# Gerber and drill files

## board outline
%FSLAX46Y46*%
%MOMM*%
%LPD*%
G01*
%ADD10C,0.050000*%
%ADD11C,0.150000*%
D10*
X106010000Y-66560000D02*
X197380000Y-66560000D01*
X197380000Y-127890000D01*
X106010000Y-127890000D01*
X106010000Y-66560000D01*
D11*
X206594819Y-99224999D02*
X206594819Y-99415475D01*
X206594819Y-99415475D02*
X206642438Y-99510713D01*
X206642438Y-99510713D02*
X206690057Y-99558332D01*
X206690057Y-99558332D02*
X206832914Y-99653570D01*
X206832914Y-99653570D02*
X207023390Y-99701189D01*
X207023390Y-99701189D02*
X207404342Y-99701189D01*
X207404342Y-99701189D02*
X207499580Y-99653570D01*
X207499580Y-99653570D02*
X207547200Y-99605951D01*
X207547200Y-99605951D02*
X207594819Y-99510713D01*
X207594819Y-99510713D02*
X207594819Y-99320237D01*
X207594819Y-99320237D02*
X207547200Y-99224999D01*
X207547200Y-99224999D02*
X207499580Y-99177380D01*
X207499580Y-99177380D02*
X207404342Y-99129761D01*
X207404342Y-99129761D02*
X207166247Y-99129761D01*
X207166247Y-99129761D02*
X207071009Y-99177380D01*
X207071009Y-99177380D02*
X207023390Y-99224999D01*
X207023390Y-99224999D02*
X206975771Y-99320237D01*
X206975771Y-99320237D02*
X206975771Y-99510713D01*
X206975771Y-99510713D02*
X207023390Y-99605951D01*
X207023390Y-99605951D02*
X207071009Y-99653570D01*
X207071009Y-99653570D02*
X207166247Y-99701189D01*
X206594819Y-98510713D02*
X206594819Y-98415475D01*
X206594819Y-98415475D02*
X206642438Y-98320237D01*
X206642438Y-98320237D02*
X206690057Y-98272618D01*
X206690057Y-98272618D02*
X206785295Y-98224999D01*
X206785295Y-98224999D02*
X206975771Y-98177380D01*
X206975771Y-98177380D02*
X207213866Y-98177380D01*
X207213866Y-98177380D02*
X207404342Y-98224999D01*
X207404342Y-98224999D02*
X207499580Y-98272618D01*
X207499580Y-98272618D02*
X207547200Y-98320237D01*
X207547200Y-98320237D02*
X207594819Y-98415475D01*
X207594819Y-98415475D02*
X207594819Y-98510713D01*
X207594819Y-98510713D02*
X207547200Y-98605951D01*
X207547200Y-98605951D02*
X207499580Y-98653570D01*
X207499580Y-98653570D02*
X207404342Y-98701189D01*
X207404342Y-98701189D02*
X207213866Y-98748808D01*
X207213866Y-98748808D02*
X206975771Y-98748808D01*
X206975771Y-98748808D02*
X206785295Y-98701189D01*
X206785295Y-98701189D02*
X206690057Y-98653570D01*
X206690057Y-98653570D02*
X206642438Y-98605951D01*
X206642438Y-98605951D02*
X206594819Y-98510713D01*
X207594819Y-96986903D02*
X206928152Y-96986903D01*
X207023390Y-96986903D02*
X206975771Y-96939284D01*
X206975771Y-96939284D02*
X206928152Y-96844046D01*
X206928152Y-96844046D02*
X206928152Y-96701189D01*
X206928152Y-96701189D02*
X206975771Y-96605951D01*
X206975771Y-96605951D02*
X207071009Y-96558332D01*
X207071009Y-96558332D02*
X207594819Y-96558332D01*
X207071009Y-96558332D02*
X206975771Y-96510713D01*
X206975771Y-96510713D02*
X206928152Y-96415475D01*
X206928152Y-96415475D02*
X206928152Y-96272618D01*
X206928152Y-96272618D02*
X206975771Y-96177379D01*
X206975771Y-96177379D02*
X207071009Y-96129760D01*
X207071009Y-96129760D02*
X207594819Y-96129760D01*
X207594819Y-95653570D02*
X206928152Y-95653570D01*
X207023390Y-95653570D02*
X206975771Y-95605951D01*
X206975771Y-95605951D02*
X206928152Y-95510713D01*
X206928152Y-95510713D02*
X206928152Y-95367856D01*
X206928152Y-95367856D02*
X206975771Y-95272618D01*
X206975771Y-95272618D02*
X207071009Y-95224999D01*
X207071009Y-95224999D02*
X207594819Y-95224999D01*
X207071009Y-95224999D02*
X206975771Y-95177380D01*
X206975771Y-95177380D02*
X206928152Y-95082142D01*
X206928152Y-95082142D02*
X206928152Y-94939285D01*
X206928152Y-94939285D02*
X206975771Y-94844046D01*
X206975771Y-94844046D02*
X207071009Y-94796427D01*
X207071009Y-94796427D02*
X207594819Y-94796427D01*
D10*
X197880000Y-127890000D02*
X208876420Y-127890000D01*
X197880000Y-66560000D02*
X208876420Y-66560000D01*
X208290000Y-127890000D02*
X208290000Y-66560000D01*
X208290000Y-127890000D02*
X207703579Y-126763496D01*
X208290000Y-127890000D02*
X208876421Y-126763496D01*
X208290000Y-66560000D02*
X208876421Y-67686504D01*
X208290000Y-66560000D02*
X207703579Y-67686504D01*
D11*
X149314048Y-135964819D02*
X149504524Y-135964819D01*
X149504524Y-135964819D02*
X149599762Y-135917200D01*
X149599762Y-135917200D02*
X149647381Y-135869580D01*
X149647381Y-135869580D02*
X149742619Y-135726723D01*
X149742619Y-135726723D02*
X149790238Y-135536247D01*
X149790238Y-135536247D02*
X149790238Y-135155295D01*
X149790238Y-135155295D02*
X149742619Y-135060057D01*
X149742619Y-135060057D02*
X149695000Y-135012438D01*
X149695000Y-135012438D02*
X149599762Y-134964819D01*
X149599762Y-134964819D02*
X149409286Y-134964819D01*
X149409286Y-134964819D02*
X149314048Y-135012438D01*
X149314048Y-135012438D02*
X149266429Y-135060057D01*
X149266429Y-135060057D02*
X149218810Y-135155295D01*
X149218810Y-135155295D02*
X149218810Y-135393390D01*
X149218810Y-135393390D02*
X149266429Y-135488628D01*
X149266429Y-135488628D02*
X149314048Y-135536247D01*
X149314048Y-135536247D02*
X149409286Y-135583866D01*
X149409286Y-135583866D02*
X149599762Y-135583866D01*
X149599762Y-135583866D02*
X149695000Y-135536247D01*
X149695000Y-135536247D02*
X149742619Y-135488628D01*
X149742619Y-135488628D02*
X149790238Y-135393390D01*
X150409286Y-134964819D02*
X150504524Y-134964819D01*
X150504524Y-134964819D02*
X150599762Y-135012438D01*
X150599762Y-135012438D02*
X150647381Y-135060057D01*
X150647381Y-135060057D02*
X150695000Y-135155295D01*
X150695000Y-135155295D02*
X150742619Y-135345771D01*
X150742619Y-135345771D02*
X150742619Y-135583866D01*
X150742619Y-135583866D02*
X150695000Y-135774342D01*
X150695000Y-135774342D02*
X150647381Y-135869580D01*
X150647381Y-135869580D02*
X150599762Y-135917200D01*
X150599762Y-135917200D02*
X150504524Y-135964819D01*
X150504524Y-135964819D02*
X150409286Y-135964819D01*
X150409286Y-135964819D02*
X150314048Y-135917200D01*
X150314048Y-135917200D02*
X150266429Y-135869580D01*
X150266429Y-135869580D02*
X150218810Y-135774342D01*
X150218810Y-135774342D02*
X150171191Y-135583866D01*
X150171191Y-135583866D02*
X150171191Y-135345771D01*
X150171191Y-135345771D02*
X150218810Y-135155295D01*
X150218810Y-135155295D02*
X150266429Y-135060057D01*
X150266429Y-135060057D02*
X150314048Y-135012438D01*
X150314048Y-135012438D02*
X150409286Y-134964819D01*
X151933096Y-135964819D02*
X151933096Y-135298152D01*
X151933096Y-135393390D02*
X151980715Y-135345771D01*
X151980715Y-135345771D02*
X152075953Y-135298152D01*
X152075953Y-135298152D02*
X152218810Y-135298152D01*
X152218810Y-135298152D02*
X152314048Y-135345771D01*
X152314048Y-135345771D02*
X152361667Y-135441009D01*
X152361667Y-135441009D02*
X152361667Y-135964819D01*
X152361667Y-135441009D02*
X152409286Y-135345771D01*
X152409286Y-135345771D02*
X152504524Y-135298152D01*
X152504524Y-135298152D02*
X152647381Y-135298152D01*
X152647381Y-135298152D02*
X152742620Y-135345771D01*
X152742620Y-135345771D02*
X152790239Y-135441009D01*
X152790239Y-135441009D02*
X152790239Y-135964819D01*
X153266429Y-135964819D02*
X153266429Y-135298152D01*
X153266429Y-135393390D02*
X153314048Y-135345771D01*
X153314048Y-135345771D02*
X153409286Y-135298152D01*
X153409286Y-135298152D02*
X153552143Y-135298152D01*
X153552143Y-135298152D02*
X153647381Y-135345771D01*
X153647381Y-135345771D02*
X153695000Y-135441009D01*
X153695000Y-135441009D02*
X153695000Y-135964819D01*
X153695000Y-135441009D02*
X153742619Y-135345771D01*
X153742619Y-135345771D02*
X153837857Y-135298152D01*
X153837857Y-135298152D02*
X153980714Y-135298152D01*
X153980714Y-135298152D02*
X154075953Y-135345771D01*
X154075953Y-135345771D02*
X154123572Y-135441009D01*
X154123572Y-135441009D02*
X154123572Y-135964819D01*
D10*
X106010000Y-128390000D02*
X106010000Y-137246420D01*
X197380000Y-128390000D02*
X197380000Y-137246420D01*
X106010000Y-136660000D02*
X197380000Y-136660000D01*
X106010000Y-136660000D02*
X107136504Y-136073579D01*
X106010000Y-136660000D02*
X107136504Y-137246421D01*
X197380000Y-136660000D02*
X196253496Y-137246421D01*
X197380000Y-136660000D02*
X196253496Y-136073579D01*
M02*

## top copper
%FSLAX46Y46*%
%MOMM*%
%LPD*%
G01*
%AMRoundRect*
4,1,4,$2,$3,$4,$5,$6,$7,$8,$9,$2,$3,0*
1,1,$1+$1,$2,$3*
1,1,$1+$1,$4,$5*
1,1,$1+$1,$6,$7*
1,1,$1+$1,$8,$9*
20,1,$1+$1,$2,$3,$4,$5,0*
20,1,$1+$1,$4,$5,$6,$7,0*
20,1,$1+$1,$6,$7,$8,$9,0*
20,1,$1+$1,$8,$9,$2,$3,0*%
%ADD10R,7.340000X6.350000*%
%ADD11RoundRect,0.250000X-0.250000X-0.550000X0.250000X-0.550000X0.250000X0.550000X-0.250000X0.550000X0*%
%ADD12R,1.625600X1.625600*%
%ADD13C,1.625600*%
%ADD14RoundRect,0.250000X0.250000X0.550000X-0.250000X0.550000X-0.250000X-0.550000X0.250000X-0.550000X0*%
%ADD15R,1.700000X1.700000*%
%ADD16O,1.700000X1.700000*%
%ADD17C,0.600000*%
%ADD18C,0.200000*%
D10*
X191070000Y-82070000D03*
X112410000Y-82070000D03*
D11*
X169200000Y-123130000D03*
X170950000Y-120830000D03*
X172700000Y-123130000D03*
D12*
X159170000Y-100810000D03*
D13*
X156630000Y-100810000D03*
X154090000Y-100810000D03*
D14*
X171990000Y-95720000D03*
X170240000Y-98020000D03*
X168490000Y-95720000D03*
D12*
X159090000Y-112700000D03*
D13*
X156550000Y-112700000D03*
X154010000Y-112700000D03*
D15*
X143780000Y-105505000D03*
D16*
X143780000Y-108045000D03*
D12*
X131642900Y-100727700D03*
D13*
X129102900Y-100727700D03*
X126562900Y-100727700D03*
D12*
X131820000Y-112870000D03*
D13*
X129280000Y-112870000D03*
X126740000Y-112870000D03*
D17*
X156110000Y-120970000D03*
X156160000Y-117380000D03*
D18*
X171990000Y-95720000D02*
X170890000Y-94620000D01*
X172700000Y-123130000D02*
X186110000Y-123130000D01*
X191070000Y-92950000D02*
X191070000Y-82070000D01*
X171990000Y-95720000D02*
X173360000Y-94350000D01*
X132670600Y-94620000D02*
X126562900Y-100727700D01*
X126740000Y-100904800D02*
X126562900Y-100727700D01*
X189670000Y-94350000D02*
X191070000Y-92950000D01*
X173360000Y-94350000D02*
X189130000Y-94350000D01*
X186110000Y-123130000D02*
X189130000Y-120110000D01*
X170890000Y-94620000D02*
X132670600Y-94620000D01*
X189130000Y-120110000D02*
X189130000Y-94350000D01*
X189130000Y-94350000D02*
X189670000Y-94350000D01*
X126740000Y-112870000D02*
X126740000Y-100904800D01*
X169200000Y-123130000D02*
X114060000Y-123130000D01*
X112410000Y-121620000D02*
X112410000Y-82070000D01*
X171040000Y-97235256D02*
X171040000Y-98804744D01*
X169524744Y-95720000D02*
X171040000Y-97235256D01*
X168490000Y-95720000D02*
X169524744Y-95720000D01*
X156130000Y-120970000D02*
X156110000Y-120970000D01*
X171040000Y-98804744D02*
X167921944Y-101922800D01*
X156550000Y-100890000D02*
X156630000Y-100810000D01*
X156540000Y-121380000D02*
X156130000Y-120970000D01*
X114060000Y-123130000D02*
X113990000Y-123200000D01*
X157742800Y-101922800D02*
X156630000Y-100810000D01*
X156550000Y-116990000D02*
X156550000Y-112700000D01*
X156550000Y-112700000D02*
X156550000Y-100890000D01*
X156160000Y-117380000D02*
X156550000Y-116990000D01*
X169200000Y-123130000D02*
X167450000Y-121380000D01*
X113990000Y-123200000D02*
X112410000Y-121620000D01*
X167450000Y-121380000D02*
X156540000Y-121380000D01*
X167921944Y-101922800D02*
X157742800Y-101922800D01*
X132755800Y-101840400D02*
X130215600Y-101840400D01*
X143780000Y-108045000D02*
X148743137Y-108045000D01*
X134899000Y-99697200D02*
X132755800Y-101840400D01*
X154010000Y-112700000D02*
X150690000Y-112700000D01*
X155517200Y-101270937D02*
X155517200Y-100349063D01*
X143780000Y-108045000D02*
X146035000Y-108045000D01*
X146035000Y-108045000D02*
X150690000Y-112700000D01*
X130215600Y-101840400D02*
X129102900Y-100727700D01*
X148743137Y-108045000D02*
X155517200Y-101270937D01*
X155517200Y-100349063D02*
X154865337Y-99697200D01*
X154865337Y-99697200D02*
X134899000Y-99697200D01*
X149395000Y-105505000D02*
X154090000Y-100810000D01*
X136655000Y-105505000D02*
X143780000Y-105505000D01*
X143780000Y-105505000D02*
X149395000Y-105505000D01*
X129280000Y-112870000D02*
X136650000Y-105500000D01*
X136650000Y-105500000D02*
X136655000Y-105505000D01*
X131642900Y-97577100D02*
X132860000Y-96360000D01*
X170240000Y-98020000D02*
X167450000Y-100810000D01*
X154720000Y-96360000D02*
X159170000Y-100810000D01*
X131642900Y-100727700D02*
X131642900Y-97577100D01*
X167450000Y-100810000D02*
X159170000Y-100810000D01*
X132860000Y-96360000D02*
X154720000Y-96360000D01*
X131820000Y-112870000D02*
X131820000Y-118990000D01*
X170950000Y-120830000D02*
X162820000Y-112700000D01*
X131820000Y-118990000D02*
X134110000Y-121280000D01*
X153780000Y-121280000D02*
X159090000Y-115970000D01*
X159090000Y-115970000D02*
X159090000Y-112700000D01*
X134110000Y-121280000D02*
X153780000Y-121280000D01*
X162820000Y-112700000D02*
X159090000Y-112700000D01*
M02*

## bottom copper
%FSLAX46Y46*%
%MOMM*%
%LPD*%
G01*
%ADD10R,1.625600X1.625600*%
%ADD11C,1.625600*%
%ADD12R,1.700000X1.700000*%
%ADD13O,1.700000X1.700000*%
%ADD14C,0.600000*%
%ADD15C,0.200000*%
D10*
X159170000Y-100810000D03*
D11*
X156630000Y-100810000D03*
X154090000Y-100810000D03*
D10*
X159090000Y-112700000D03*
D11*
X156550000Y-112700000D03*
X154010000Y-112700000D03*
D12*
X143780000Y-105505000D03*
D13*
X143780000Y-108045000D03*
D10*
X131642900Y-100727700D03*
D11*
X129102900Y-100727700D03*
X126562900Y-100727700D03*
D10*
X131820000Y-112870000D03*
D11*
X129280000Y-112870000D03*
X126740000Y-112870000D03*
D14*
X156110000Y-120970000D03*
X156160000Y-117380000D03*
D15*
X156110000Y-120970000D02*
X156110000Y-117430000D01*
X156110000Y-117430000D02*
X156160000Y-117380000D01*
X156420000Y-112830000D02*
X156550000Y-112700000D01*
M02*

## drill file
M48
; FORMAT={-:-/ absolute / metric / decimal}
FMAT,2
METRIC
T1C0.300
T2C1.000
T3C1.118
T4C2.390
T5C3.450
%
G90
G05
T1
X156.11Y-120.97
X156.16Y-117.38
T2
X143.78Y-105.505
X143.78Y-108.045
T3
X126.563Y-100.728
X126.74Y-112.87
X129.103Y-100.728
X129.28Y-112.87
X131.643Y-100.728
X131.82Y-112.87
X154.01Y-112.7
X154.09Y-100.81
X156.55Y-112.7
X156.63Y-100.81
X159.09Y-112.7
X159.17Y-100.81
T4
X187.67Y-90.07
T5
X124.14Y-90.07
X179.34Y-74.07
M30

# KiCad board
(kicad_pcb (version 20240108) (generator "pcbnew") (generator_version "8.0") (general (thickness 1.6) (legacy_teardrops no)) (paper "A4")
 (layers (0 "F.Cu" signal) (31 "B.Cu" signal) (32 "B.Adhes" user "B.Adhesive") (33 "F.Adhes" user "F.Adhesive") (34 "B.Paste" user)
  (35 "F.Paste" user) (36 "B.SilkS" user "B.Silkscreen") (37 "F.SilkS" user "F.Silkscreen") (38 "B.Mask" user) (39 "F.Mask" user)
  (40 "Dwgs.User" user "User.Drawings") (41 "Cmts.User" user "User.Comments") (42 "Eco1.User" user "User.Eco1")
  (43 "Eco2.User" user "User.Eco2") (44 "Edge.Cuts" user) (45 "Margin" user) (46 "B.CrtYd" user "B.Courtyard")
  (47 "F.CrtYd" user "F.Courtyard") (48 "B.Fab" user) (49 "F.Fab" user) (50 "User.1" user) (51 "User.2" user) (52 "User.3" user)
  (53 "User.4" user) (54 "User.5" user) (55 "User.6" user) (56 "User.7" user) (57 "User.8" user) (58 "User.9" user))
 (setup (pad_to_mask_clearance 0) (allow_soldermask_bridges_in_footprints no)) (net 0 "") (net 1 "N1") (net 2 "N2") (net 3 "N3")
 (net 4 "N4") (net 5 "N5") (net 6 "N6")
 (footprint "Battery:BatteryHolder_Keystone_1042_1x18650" (layer "F.Cu") (at 151.74 82.07 180)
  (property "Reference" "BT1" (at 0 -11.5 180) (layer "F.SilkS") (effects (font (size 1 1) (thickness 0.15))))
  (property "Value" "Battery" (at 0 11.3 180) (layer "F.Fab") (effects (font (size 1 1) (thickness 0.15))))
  (pad "" np_thru_hole circle (at -35.93 -8 180) (size 2.39 2.39) (drill 2.39) (layers "*.Cu" "*.Mask"))
  (pad "" np_thru_hole circle (at -27.6 8 180) (size 3.45 3.45) (drill 3.45) (layers "*.Cu" "*.Mask"))
  (pad "" np_thru_hole circle (at 27.6 -8 180) (size 3.45 3.45) (drill 3.45) (layers "*.Cu" "*.Mask"))
  (pad "1" smd rect (at -39.33 0 180) (size 7.34 6.35) (layers "F.Cu" "F.Paste" "F.Mask") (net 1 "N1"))
  (pad "2" smd rect (at 39.33 0 180) (size 7.34 6.35) (layers "F.Cu" "F.Paste" "F.Mask") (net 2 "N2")))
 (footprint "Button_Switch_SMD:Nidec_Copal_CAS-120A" (layer "F.Cu") (at 170.95 121.98 90)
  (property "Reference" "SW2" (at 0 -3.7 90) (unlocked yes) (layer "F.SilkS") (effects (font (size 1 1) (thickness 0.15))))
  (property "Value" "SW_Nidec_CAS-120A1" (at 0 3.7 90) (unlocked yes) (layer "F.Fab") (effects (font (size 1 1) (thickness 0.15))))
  (pad "1" smd roundrect (at -1.15 -1.75) (size 1 1.6) (layers "F.Cu" "F.Paste" "F.Mask") (roundrect_rratio 0.25) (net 2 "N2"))
  (pad "2" smd roundrect (at 1.15 0) (size 1 1.6) (layers "F.Cu" "F.Paste" "F.Mask") (roundrect_rratio 0.25) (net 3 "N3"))
  (pad "3" smd roundrect (at -1.15 1.75) (size 1 1.6) (layers "F.Cu" "F.Paste" "F.Mask") (roundrect_rratio 0.25) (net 1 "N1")))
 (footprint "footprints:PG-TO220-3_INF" (layer "F.Cu") (at 159.17 100.81 180)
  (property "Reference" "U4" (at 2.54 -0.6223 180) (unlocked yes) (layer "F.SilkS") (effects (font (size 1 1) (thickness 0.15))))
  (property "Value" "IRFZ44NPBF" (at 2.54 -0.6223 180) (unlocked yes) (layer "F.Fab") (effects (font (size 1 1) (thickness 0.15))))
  (pad "1" thru_hole rect (at 0 0 180) (size 1.6256 1.6256) (drill 1.1176) (layers "*.Cu" "*.Mask") (remove_unused_layers no) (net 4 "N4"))
  (pad "2" thru_hole circle (at 2.54 0 180) (size 1.6256 1.6256) (drill 1.1176) (layers "*.Cu" "*.Mask") (remove_unused_layers no)
   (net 2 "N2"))
  (pad "3" thru_hole circle (at 5.08 0 180) (size 1.6256 1.6256) (drill 1.1176) (layers "*.Cu" "*.Mask") (remove_unused_layers no)
   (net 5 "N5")))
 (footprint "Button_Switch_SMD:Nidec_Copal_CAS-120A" (layer "F.Cu") (at 170.24 96.87 -90)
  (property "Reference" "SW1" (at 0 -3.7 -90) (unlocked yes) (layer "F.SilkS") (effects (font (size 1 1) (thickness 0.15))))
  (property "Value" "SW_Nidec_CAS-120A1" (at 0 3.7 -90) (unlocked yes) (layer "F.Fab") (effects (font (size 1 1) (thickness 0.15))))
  (pad "1" smd roundrect (at -1.15 -1.75 180) (size 1 1.6) (layers "F.Cu" "F.Paste" "F.Mask") (roundrect_rratio 0.25) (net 1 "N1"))
  (pad "2" smd roundrect (at 1.15 0 180) (size 1 1.6) (layers "F.Cu" "F.Paste" "F.Mask") (roundrect_rratio 0.25) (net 4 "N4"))
  (pad "3" smd roundrect (at -1.15 1.75 180) (size 1 1.6) (layers "F.Cu" "F.Paste" "F.Mask") (roundrect_rratio 0.25) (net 2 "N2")))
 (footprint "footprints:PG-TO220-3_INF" (layer "F.Cu") (at 159.09 112.7 180)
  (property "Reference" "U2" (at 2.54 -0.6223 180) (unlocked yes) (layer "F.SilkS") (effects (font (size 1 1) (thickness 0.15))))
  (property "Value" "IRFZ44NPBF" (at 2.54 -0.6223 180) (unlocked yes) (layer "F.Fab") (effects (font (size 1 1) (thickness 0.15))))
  (pad "1" thru_hole rect (at 0 0 180) (size 1.6256 1.6256) (drill 1.1176) (layers "*.Cu" "*.Mask") (remove_unused_layers no) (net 3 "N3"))
  (pad "2" thru_hole circle (at 2.54 0 180) (size 1.6256 1.6256) (drill 1.1176) (layers "*.Cu" "*.Mask") (remove_unused_layers no)
   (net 2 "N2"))
  (pad "3" thru_hole circle (at 5.08 0 180) (size 1.6256 1.6256) (drill 1.1176) (layers "*.Cu" "*.Mask") (remove_unused_layers no)
   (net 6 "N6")))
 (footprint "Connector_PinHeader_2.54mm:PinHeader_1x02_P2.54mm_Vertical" (layer "F.Cu") (at 143.78 105.505)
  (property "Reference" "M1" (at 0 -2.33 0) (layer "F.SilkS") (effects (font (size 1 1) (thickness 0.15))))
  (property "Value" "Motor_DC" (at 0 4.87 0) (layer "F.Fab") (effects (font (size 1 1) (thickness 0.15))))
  (pad "1" thru_hole rect (at 0 0) (size 1.7 1.7) (drill 1) (layers "*.Cu" "*.Mask") (remove_unused_layers no) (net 5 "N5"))
  (pad "2" thru_hole oval (at 0 2.54) (size 1.7 1.7) (drill 1) (layers "*.Cu" "*.Mask") (remove_unused_layers no) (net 6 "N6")))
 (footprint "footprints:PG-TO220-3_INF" (layer "F.Cu") (at 131.6429 100.7277 180)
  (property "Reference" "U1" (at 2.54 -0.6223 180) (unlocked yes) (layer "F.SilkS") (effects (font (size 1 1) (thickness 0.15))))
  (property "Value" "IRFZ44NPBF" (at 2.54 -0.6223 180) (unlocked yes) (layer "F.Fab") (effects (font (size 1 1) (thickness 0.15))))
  (pad "1" thru_hole rect (at 0 0 180) (size 1.6256 1.6256) (drill 1.1176) (layers "*.Cu" "*.Mask") (remove_unused_layers no) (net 4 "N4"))
  (pad "2" thru_hole circle (at 2.54 0 180) (size 1.6256 1.6256) (drill 1.1176) (layers "*.Cu" "*.Mask") (remove_unused_layers no)
   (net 6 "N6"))
  (pad "3" thru_hole circle (at 5.08 0 180) (size 1.6256 1.6256) (drill 1.1176) (layers "*.Cu" "*.Mask") (remove_unused_layers no)
   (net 1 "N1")))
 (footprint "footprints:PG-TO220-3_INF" (layer "F.Cu") (at 131.82 112.87 180)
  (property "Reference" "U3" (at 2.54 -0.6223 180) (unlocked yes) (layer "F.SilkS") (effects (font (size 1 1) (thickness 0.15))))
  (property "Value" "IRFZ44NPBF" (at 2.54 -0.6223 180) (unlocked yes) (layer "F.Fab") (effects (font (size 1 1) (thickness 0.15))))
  (pad "1" thru_hole rect (at 0 0 180) (size 1.6256 1.6256) (drill 1.1176) (layers "*.Cu" "*.Mask") (remove_unused_layers no) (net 3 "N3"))
  (pad "2" thru_hole circle (at 2.54 0 180) (size 1.6256 1.6256) (drill 1.1176) (layers "*.Cu" "*.Mask") (remove_unused_layers no)
   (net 5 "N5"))
  (pad "3" thru_hole circle (at 5.08 0 180) (size 1.6256 1.6256) (drill 1.1176) (layers "*.Cu" "*.Mask") (remove_unused_layers no)
   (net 1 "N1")))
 (gr_rect (start 106.01 66.56) (end 197.38 127.89) (stroke (width 0.05) (type default)) (fill none) (layer "Edge.Cuts"))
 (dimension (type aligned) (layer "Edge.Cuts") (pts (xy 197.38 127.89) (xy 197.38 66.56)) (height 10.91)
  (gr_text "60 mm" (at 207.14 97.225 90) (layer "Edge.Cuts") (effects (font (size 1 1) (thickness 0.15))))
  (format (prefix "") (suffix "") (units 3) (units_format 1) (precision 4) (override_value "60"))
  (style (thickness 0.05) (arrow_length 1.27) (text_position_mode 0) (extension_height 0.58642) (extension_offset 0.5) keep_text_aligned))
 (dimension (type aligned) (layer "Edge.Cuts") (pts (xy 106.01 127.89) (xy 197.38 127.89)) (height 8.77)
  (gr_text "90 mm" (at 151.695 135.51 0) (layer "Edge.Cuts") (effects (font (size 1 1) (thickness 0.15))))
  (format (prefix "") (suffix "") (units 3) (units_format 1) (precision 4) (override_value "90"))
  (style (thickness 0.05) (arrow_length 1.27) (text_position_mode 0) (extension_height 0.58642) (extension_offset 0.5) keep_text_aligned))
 (segment (start 171.99 95.72) (end 170.89 94.62) (width 0.2) (layer "F.Cu") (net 1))
 (segment (start 172.7 123.13) (end 186.11 123.13) (width 0.2) (layer "F.Cu") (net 1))
 (segment (start 191.07 92.95) (end 191.07 82.07) (width 0.2) (layer "F.Cu") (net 1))
 (segment (start 171.99 95.72) (end 173.36 94.35) (width 0.2) (layer "F.Cu") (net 1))
 (segment (start 132.6706 94.62) (end 126.5629 100.7277) (width 0.2) (layer "F.Cu") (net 1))
 (segment (start 126.74 100.9048) (end 126.5629 100.7277) (width 0.2) (layer "F.Cu") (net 1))
 (segment (start 189.67 94.35) (end 191.07 92.95) (width 0.2) (layer "F.Cu") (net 1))
 (segment (start 173.36 94.35) (end 189.13 94.35) (width 0.2) (layer "F.Cu") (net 1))
 (segment (start 186.11 123.13) (end 189.13 120.11) (width 0.2) (layer "F.Cu") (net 1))
 (segment (start 170.89 94.62) (end 132.6706 94.62) (width 0.2) (layer "F.Cu") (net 1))
 (segment (start 189.13 120.11) (end 189.13 94.35) (width 0.2) (layer "F.Cu") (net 1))
 (segment (start 189.13 94.35) (end 189.67 94.35) (width 0.2) (layer "F.Cu") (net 1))
 (segment (start 126.74 112.87) (end 126.74 100.9048) (width 0.2) (layer "F.Cu") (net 1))
 (segment (start 169.2 123.13) (end 114.06 123.13) (width 0.2) (layer "F.Cu") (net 2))
 (segment (start 112.41 121.62) (end 112.41 82.07) (width 0.2) (layer "F.Cu") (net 2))
 (segment (start 171.04 97.235256) (end 171.04 98.804744) (width 0.2) (layer "F.Cu") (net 2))
 (segment (start 169.524744 95.72) (end 171.04 97.235256) (width 0.2) (layer "F.Cu") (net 2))
 (segment (start 168.49 95.72) (end 169.524744 95.72) (width 0.2) (layer "F.Cu") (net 2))
 (segment (start 156.13 120.97) (end 156.11 120.97) (width 0.2) (layer "F.Cu") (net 2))
 (segment (start 171.04 98.804744) (end 167.921944 101.9228) (width 0.2) (layer "F.Cu") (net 2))
 (segment (start 156.55 100.89) (end 156.63 100.81) (width 0.2) (layer "F.Cu") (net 2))
 (segment (start 156.54 121.38) (end 156.13 120.97) (width 0.2) (layer "F.Cu") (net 2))
 (segment (start 114.06 123.13) (end 113.99 123.2) (width 0.2) (layer "F.Cu") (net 2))
 (segment (start 157.7428 101.9228) (end 156.63 100.81) (width 0.2) (layer "F.Cu") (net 2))
 (segment (start 156.55 116.99) (end 156.55 112.7) (width 0.2) (layer "F.Cu") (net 2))
 (segment (start 156.55 112.7) (end 156.55 100.89) (width 0.2) (layer "F.Cu") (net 2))
 (segment (start 156.16 117.38) (end 156.55 116.99) (width 0.2) (layer "F.Cu") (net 2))
 (segment (start 169.2 123.13) (end 167.45 121.38) (width 0.2) (layer "F.Cu") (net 2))
 (segment (start 113.99 123.2) (end 112.41 121.62) (width 0.2) (layer "F.Cu") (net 2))
 (segment (start 167.45 121.38) (end 156.54 121.38) (width 0.2) (layer "F.Cu") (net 2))
 (segment (start 167.921944 101.9228) (end 157.7428 101.9228) (width 0.2) (layer "F.Cu") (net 2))
 (via (at 156.11 120.97) (size 0.6) (drill 0.3) (layers "F.Cu" "B.Cu") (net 2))
 (via (at 156.16 117.38) (size 0.6) (drill 0.3) (layers "F.Cu" "B.Cu") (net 2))
 (segment (start 156.11 120.97) (end 156.11 117.43) (width 0.2) (layer "B.Cu") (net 2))
 (segment (start 156.11 117.43) (end 156.16 117.38) (width 0.2) (layer "B.Cu") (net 2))
 (segment (start 156.42 112.83) (end 156.55 112.7) (width 0.2) (layer "B.Cu") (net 2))
 (segment (start 132.7558 101.8404) (end 130.2156 101.8404) (width 0.2) (layer "F.Cu") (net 6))
 (segment (start 143.78 108.045) (end 148.743137 108.045) (width 0.2) (layer "F.Cu") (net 6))
 (segment (start 134.899 99.6972) (end 132.7558 101.8404) (width 0.2) (layer "F.Cu") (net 6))
 (segment (start 154.01 112.7) (end 150.69 112.7) (width 0.2) (layer "F.Cu") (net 6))
 (segment (start 155.5172 101.270937) (end 155.5172 100.349063) (width 0.2) (layer "F.Cu") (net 6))
 (segment (start 143.78 108.045) (end 146.035 108.045) (width 0.2) (layer "F.Cu") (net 6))
 (segment (start 146.035 108.045) (end 150.69 112.7) (width 0.2) (layer "F.Cu") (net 6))
 (segment (start 130.2156 101.8404) (end 129.1029 100.7277) (width 0.2) (layer "F.Cu") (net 6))
 (segment (start 148.743137 108.045) (end 155.5172 101.270937) (width 0.2) (layer "F.Cu") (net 6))
 (segment (start 155.5172 100.349063) (end 154.865337 99.6972) (width 0.2) (layer "F.Cu") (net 6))
 (segment (start 154.865337 99.6972) (end 134.899 99.6972) (width 0.2) (layer "F.Cu") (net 6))
 (segment (start 149.395 105.505) (end 154.09 100.81) (width 0.2) (layer "F.Cu") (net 5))
 (segment (start 136.655 105.505) (end 143.78 105.505) (width 0.2) (layer "F.Cu") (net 5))
 (segment (start 143.78 105.505) (end 149.395 105.505) (width 0.2) (layer "F.Cu") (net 5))
 (segment (start 129.28 112.87) (end 136.65 105.5) (width 0.2) (layer "F.Cu") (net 5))
 (segment (start 136.65 105.5) (end 136.655 105.505) (width 0.2) (layer "F.Cu") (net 5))
 (segment (start 131.6429 97.5771) (end 132.86 96.36) (width 0.2) (layer "F.Cu") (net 4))
 (segment (start 170.24 98.02) (end 167.45 100.81) (width 0.2) (layer "F.Cu") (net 4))
 (segment (start 154.72 96.36) (end 159.17 100.81) (width 0.2) (layer "F.Cu") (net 4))
 (segment (start 131.6429 100.7277) (end 131.6429 97.5771) (width 0.2) (layer "F.Cu") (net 4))
 (segment (start 167.45 100.81) (end 159.17 100.81) (width 0.2) (layer "F.Cu") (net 4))
 (segment (start 132.86 96.36) (end 154.72 96.36) (width 0.2) (layer "F.Cu") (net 4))
 (segment (start 131.82 112.87) (end 131.82 118.99) (width 0.2) (layer "F.Cu") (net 3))
 (segment (start 170.95 120.83) (end 162.82 112.7) (width 0.2) (layer "F.Cu") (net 3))
 (segment (start 131.82 118.99) (end 134.11 121.28) (width 0.2) (layer "F.Cu") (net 3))
 (segment (start 153.78 121.28) (end 159.09 115.97) (width 0.2) (layer "F.Cu") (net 3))
 (segment (start 159.09 115.97) (end 159.09 112.7) (width 0.2) (layer "F.Cu") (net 3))
 (segment (start 134.11 121.28) (end 153.78 121.28) (width 0.2) (layer "F.Cu") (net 3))
 (segment (start 162.82 112.7) (end 159.09 112.7) (width 0.2) (layer "F.Cu") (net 3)))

